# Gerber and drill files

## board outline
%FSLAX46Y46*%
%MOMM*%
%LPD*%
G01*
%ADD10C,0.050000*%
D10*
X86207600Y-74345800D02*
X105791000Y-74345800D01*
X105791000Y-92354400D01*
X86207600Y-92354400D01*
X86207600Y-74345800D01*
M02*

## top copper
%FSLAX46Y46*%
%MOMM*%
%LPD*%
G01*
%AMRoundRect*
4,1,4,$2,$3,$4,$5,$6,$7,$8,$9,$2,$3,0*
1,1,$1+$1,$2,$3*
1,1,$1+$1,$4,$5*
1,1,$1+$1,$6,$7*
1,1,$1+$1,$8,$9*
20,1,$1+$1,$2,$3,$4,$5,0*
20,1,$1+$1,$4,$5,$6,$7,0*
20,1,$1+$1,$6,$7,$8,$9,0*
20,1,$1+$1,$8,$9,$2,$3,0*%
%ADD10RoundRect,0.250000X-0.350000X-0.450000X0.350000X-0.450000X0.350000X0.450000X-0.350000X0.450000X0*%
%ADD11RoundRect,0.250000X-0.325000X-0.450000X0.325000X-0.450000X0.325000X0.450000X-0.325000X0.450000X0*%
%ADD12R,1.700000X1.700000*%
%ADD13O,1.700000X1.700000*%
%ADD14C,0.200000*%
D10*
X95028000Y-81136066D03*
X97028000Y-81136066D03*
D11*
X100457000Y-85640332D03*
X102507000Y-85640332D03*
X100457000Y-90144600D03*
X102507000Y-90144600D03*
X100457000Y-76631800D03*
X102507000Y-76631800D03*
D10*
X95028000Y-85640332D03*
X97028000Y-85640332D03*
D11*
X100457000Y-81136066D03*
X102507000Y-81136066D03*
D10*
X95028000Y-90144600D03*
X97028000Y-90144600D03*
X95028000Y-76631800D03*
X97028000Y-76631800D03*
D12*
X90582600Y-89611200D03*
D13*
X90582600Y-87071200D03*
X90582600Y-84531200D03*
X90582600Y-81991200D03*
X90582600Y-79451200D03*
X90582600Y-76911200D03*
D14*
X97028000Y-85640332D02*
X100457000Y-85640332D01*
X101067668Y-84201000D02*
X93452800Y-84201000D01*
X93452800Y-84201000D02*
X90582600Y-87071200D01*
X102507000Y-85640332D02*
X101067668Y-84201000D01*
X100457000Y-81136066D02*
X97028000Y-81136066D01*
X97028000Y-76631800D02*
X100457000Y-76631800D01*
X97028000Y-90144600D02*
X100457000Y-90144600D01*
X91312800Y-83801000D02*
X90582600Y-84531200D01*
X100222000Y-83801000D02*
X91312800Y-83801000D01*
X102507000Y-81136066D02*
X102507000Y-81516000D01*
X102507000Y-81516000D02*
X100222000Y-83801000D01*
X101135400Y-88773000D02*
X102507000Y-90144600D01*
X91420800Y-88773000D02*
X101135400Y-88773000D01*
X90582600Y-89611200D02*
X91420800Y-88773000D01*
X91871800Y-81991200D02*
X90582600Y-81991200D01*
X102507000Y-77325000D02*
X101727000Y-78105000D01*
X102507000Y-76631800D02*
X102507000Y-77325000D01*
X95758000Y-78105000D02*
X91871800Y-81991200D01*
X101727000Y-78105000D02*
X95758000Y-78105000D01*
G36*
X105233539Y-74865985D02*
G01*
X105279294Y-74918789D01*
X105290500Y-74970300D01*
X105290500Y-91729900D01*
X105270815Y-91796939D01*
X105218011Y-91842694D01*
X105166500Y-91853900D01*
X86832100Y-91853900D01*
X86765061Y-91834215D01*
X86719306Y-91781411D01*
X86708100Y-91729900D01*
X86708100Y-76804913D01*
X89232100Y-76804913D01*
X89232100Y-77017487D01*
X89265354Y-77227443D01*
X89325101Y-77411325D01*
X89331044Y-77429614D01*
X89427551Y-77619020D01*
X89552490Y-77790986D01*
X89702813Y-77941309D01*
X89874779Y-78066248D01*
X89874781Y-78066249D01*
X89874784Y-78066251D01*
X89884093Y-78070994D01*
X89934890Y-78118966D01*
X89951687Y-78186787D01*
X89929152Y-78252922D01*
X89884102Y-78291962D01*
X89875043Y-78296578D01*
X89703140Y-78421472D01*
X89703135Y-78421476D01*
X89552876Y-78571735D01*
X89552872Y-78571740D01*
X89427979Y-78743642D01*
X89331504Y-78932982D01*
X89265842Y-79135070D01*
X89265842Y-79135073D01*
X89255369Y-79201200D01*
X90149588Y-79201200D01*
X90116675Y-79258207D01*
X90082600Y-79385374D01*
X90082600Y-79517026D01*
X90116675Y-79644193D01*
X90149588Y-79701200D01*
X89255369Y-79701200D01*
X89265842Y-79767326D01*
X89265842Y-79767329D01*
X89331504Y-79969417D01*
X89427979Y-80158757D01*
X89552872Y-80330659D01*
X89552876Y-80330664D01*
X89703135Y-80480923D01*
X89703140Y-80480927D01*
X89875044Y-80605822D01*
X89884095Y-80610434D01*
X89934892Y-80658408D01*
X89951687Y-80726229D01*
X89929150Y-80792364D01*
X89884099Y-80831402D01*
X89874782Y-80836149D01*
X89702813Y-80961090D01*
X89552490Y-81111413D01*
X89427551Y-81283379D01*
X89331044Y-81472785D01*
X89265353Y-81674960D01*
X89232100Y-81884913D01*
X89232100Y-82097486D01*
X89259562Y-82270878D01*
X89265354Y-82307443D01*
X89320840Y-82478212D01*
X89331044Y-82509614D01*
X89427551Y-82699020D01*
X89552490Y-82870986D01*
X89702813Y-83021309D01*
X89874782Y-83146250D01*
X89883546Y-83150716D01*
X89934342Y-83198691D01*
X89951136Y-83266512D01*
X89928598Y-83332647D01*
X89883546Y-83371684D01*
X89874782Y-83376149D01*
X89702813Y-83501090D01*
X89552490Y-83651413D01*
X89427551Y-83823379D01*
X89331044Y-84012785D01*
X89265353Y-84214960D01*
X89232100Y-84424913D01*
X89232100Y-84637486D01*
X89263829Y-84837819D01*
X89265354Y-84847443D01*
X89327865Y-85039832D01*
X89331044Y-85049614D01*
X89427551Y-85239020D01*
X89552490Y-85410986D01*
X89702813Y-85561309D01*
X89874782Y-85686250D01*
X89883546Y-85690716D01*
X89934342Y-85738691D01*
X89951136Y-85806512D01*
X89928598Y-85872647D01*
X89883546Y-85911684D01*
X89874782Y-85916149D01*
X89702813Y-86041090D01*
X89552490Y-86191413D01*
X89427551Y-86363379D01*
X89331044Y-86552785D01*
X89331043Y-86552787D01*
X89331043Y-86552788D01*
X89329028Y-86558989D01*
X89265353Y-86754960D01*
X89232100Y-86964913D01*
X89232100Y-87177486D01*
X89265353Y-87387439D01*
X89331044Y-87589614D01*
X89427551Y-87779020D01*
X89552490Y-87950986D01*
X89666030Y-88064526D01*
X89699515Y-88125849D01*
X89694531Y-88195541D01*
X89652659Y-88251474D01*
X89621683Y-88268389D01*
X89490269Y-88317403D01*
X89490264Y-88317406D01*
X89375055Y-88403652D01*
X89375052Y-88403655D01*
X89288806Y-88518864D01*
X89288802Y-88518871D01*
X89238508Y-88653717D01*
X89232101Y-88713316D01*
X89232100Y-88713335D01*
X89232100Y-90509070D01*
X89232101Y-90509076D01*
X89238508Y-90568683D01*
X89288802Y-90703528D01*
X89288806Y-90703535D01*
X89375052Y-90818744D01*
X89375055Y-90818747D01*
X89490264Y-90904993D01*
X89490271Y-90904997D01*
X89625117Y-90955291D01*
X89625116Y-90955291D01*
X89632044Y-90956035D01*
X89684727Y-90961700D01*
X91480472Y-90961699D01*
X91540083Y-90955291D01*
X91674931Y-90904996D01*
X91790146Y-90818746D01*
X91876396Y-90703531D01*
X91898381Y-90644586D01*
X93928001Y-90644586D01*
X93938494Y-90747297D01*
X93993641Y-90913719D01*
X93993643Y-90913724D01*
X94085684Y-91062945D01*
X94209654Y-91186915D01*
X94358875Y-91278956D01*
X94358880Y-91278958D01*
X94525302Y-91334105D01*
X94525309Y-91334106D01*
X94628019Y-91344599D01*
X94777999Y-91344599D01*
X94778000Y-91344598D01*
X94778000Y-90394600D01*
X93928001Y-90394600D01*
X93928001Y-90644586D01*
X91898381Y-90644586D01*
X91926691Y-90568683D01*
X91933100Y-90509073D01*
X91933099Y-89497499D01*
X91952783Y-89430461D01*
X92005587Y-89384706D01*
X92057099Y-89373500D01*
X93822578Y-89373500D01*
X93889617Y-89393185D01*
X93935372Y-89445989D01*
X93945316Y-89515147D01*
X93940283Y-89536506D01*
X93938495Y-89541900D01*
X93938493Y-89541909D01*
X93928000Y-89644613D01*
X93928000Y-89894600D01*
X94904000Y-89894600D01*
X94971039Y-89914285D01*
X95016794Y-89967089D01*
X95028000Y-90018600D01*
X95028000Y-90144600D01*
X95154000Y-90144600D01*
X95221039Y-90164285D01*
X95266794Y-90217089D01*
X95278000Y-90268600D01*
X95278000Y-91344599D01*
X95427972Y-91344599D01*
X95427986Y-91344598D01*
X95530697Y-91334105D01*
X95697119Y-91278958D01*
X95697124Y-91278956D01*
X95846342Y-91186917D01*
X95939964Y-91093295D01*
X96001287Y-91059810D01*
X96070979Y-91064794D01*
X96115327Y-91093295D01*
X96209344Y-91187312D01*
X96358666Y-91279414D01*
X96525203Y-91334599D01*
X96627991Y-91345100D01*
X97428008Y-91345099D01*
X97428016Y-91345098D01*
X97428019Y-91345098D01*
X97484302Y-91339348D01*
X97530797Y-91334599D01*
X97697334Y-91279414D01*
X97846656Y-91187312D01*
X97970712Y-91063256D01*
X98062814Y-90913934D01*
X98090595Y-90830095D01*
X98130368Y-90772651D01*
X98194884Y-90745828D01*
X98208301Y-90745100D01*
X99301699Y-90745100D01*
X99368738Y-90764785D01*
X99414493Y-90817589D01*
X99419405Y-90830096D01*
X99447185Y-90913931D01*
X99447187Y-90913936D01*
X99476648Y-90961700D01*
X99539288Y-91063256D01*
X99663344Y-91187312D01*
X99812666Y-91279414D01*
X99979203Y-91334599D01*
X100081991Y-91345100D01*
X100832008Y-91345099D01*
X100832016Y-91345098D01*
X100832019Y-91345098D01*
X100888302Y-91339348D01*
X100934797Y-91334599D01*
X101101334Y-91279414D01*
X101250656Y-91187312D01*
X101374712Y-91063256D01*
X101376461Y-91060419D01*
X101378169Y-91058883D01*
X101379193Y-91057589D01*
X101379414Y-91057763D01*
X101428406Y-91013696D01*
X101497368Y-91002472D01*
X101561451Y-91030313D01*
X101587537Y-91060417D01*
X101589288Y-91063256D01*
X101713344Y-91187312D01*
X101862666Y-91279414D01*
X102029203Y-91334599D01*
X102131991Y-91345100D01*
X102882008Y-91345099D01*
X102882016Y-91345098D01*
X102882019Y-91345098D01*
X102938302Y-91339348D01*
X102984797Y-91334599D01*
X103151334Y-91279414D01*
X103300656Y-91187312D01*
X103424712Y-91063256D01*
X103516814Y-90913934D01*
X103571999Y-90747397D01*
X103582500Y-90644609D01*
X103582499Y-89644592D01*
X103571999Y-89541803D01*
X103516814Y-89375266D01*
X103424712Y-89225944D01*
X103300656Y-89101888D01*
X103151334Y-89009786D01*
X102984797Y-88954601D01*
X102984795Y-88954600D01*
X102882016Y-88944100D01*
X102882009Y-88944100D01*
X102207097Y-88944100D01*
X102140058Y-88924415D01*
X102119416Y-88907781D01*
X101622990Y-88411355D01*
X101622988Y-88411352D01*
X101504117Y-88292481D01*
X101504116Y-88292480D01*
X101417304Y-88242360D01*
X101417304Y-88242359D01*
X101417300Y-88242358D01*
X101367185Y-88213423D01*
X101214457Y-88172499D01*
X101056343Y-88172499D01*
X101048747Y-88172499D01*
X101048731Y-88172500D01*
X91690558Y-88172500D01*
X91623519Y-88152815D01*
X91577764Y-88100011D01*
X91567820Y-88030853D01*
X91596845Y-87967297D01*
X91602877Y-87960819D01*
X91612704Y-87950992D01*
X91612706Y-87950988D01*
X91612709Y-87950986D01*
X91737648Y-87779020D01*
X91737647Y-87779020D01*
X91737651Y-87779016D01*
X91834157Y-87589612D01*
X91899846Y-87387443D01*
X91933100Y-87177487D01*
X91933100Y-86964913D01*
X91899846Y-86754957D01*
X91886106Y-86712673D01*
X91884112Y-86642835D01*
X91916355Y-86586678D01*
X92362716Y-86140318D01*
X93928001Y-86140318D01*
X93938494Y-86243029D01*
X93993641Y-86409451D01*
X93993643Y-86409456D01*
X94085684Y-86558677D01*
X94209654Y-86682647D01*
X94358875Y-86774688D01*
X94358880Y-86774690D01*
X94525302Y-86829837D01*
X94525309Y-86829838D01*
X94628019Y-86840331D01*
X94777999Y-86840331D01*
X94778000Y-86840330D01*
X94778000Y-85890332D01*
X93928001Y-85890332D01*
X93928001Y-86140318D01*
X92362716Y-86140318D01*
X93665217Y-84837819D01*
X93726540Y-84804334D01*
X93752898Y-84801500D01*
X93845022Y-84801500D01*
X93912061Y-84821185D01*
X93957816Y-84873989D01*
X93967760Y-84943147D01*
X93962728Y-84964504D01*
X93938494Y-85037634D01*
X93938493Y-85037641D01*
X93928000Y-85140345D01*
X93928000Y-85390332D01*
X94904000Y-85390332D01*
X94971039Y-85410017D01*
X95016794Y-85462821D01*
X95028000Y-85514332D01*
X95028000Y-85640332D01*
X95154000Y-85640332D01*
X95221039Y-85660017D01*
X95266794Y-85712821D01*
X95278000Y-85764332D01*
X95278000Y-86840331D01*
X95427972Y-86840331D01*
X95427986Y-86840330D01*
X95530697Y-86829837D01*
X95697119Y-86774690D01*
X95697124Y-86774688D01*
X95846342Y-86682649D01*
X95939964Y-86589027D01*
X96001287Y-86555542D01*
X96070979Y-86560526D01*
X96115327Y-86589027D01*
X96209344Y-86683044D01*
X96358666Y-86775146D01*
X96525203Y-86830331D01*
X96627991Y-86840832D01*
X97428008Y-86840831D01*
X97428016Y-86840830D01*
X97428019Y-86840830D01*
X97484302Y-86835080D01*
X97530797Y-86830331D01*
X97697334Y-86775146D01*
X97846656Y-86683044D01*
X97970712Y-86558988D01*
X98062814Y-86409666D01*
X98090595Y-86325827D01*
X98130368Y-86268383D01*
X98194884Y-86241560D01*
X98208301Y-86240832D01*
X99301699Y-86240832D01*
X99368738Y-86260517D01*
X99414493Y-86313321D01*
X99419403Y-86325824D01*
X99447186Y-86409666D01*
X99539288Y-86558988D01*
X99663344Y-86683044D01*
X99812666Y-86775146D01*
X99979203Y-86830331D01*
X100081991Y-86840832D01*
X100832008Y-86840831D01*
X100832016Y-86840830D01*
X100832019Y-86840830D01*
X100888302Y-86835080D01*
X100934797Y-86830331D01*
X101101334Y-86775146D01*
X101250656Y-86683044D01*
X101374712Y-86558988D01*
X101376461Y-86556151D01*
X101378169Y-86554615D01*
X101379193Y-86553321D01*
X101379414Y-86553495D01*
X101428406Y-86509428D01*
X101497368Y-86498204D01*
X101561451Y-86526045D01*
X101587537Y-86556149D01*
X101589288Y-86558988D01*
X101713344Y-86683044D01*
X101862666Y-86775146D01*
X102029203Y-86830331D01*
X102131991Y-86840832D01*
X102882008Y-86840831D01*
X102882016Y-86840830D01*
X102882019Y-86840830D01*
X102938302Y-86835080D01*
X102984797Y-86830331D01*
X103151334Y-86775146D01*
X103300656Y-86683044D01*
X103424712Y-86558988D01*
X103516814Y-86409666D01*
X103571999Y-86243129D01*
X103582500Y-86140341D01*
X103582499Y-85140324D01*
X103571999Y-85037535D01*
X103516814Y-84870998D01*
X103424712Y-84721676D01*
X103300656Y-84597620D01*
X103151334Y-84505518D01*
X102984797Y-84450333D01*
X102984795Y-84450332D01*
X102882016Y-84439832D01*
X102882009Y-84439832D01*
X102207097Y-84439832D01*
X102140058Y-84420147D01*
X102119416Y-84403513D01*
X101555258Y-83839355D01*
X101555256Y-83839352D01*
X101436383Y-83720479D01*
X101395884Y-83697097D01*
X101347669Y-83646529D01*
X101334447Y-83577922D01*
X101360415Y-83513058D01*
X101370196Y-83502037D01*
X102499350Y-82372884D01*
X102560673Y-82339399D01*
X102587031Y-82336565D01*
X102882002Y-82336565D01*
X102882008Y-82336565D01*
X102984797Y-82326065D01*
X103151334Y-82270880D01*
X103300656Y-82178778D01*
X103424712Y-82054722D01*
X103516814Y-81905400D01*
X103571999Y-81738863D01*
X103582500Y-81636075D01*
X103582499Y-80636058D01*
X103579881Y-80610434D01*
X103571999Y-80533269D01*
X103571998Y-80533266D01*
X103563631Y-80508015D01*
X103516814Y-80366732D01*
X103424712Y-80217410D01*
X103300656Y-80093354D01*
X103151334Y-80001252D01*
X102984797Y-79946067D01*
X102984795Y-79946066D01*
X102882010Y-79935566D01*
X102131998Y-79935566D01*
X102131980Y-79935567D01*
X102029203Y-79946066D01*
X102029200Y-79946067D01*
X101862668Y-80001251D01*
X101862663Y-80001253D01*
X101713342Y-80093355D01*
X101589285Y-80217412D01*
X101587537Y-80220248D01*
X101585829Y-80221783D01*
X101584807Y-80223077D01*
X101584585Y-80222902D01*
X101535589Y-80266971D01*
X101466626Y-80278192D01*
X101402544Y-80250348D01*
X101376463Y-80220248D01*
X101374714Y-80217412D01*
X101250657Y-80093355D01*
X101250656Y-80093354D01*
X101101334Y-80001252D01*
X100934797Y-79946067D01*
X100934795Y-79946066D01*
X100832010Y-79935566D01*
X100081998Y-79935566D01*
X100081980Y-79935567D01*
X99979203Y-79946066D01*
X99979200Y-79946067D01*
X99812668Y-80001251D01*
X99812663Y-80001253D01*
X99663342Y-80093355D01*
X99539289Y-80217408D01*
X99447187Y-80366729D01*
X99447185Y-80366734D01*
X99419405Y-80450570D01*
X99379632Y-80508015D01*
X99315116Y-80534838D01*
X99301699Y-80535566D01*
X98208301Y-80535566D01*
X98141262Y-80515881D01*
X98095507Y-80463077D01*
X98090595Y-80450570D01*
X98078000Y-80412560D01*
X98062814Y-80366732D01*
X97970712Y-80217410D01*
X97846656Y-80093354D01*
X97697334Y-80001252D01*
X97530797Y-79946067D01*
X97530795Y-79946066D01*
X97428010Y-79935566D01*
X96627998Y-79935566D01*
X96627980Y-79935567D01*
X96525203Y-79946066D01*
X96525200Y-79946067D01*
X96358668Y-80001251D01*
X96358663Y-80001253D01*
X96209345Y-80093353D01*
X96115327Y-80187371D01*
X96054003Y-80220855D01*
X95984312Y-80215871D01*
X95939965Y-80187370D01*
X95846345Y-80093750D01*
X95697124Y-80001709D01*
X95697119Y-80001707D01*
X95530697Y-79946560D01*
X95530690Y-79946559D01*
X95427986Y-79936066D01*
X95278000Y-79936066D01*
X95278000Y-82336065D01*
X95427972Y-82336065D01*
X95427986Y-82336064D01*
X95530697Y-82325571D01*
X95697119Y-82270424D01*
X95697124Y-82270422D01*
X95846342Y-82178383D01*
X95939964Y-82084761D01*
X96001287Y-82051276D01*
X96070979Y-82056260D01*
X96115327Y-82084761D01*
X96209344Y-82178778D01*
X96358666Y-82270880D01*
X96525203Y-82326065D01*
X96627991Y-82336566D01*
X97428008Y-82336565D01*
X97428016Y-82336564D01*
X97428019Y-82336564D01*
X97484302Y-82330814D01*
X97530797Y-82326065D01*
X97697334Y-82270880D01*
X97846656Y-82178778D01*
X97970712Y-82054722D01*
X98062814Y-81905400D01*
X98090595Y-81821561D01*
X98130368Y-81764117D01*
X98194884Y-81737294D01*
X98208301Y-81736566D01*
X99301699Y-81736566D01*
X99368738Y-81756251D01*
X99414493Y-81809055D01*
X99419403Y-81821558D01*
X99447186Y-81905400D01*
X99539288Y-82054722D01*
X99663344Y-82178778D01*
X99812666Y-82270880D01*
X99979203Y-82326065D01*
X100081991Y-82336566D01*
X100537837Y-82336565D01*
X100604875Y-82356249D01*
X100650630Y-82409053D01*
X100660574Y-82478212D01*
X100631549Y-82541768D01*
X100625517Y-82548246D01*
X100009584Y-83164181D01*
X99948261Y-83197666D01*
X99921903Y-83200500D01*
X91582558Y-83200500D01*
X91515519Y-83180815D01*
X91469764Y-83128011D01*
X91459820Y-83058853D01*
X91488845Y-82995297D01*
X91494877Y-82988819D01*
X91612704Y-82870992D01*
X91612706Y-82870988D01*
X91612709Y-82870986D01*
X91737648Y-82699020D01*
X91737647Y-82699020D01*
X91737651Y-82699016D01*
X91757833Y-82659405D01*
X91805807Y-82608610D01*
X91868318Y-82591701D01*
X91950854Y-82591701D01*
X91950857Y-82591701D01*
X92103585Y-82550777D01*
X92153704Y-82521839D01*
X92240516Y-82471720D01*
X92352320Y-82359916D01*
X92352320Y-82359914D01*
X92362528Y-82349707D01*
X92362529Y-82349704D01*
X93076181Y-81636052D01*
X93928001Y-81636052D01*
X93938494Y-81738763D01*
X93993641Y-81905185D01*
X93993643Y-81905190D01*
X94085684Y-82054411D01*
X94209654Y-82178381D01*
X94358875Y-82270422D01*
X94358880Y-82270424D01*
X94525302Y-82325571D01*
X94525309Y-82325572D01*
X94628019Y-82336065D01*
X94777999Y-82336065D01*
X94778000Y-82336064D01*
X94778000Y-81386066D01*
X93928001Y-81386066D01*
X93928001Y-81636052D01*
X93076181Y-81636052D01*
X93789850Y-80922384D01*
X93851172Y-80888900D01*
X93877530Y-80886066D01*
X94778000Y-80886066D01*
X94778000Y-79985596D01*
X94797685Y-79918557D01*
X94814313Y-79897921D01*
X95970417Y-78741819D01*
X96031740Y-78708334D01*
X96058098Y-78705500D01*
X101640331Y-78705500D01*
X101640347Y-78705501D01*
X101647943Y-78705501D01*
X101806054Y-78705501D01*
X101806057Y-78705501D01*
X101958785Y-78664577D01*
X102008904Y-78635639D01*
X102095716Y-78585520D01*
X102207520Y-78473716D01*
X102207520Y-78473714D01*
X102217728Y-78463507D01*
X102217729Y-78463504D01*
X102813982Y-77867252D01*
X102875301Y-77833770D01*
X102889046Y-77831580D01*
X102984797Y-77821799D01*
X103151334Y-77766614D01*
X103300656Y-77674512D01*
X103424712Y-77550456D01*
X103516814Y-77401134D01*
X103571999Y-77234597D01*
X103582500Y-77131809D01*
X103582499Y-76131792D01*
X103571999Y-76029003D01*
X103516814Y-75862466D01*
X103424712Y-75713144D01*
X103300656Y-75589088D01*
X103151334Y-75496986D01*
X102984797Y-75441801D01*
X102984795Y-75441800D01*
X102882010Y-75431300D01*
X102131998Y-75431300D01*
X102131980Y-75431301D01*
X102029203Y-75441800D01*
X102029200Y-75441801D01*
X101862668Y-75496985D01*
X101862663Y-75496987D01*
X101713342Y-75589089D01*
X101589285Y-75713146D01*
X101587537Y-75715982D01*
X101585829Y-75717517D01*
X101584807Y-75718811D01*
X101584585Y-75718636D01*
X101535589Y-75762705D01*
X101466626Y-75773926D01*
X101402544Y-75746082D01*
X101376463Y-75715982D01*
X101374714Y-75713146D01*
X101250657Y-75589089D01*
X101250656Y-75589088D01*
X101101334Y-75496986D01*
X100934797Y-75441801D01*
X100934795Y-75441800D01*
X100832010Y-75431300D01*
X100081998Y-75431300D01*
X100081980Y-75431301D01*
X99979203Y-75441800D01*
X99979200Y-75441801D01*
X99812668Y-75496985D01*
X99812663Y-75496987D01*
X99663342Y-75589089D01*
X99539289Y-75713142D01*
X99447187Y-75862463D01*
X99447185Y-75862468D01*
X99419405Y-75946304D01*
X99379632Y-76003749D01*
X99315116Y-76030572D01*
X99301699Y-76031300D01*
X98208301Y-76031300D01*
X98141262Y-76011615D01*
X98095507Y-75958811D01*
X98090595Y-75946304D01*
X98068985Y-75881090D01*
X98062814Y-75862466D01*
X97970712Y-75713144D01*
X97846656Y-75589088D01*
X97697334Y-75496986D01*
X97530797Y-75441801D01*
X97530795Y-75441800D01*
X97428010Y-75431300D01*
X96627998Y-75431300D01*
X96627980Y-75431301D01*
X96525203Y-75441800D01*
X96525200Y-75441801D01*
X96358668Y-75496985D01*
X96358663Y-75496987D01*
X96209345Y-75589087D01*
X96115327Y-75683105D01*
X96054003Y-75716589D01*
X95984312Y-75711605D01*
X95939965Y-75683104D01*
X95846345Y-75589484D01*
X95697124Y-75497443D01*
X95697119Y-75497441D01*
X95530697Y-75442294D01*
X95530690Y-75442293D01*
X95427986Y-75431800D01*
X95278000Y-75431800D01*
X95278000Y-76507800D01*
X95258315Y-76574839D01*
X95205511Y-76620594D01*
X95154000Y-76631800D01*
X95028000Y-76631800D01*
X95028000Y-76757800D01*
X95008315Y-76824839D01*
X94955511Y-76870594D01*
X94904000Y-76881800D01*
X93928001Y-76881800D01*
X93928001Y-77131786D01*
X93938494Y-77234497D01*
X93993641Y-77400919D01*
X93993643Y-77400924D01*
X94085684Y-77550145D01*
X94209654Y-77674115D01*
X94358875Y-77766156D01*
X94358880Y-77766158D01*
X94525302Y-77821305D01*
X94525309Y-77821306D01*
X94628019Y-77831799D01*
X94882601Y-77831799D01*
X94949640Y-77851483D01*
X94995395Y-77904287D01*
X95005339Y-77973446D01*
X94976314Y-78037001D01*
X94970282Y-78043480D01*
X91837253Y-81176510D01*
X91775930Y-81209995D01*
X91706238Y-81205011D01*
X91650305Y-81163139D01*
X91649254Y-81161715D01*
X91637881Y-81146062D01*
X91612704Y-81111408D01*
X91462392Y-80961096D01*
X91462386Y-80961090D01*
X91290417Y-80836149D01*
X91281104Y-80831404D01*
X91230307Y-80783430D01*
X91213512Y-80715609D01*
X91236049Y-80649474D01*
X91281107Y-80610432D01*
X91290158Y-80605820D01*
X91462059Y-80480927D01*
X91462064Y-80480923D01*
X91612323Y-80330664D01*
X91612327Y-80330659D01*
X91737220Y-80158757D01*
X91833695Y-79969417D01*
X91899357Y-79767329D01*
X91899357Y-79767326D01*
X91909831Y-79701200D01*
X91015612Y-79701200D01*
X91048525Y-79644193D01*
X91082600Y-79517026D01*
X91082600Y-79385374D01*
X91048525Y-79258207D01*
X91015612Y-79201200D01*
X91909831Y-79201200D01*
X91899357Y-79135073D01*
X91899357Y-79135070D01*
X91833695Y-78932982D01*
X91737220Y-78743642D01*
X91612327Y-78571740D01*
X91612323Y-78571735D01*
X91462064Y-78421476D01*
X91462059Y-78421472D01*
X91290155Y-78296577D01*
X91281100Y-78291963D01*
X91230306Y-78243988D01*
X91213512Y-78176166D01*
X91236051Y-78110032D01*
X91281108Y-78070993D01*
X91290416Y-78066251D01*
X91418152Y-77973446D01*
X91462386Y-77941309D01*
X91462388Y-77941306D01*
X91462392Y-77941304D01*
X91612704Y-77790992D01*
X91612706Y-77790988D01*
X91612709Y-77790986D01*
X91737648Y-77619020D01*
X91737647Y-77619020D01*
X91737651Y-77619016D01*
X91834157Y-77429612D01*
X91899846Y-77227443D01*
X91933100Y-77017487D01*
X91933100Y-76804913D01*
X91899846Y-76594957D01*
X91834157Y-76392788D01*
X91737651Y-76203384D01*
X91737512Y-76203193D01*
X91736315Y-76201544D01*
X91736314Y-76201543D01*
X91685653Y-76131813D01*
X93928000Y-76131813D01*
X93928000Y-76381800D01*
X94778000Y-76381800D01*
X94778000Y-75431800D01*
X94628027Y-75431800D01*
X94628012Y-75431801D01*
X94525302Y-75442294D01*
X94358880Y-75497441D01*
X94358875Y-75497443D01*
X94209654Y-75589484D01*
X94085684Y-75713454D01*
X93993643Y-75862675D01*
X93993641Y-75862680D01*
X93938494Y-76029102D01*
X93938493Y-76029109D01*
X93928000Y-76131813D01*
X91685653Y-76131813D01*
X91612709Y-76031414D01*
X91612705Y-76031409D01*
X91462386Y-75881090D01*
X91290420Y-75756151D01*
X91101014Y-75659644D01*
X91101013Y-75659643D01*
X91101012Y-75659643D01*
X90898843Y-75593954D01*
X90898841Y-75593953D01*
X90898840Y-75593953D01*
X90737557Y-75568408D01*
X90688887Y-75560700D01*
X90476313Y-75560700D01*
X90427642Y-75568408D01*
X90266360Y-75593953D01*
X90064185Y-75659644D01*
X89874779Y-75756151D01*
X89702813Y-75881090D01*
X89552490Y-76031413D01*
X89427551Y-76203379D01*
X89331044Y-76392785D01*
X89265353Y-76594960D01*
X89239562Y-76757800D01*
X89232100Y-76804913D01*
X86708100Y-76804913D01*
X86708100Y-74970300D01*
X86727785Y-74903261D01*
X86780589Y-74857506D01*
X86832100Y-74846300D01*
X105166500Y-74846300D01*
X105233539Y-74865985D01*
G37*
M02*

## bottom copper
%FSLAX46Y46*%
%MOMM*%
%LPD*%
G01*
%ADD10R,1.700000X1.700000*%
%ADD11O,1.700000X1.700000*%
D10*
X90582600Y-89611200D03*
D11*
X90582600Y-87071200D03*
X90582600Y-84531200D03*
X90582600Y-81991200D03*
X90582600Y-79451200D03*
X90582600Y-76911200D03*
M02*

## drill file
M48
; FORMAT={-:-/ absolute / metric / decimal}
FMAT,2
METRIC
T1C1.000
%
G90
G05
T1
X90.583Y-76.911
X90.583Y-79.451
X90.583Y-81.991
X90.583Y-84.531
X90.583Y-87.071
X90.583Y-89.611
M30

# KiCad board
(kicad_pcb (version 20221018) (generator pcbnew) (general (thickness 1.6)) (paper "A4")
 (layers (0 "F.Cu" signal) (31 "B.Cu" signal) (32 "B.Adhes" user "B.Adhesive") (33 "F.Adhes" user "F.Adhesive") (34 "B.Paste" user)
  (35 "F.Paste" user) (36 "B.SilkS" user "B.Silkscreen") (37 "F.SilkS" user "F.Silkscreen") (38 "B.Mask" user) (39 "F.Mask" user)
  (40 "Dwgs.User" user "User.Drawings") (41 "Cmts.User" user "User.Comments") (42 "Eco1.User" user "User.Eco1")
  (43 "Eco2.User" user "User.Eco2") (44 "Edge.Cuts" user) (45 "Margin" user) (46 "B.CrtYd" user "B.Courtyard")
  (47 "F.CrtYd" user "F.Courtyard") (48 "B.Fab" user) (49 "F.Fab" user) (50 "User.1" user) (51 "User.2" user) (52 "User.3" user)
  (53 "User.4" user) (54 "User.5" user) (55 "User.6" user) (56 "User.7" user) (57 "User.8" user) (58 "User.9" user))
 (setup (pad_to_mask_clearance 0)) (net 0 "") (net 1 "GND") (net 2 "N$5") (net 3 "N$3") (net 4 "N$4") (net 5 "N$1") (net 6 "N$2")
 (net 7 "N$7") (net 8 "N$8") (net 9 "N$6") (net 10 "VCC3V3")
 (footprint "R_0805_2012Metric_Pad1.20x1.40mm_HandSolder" (layer "F.Cu") (at 96.028 81.136066)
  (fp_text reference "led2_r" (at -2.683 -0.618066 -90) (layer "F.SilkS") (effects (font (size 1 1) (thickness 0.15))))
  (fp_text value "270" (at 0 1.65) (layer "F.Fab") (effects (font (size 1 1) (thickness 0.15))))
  (pad "1" smd roundrect (at -1 0) (size 1.2 1.4) (layers "F.Cu" "F.Paste" "F.Mask") (roundrect_rratio 0.208333) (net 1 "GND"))
  (pad "2" smd roundrect (at 1 0) (size 1.2 1.4) (layers "F.Cu" "F.Paste" "F.Mask") (roundrect_rratio 0.208333) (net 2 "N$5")))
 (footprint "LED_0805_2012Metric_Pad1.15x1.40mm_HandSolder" (layer "F.Cu") (at 101.482 85.640332)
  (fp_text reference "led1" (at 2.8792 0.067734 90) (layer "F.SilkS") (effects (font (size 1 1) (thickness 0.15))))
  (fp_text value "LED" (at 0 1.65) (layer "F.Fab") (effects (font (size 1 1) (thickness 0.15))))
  (pad "1" smd roundrect (at -1.025 0) (size 1.15 1.4) (layers "F.Cu" "F.Paste" "F.Mask") (roundrect_rratio 0.217391) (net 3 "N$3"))
  (pad "2" smd roundrect (at 1.025 0) (size 1.15 1.4) (layers "F.Cu" "F.Paste" "F.Mask") (roundrect_rratio 0.217391) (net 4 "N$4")))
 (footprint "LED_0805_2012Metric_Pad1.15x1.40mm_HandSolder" (layer "F.Cu") (at 101.482 90.1446)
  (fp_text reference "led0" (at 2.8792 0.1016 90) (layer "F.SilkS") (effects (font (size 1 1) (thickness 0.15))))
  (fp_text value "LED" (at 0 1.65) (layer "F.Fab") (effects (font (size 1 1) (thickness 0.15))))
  (pad "1" smd roundrect (at -1.025 0) (size 1.15 1.4) (layers "F.Cu" "F.Paste" "F.Mask") (roundrect_rratio 0.217391) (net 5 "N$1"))
  (pad "2" smd roundrect (at 1.025 0) (size 1.15 1.4) (layers "F.Cu" "F.Paste" "F.Mask") (roundrect_rratio 0.217391) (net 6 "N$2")))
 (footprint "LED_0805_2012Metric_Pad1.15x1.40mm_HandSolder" (layer "F.Cu") (at 101.482 76.6318)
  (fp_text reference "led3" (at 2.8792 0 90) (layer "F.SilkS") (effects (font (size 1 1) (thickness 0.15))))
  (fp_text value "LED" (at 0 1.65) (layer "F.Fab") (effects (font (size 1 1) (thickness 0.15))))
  (pad "1" smd roundrect (at -1.025 0) (size 1.15 1.4) (layers "F.Cu" "F.Paste" "F.Mask") (roundrect_rratio 0.217391) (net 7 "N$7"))
  (pad "2" smd roundrect (at 1.025 0) (size 1.15 1.4) (layers "F.Cu" "F.Paste" "F.Mask") (roundrect_rratio 0.217391) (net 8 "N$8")))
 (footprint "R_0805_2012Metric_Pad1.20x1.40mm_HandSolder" (layer "F.Cu") (at 96.028 85.640332)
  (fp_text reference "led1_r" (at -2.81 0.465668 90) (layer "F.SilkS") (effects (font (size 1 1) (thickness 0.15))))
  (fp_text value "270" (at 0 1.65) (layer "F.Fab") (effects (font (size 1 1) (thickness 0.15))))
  (pad "1" smd roundrect (at -1 0) (size 1.2 1.4) (layers "F.Cu" "F.Paste" "F.Mask") (roundrect_rratio 0.208333) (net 1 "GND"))
  (pad "2" smd roundrect (at 1 0) (size 1.2 1.4) (layers "F.Cu" "F.Paste" "F.Mask") (roundrect_rratio 0.208333) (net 3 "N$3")))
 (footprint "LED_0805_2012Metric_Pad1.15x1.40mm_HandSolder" (layer "F.Cu") (at 101.482 81.136066)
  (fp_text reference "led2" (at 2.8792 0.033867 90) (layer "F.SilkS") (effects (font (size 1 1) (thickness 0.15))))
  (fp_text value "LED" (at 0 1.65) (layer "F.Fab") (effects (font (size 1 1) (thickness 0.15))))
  (pad "1" smd roundrect (at -1.025 0) (size 1.15 1.4) (layers "F.Cu" "F.Paste" "F.Mask") (roundrect_rratio 0.217391) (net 2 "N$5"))
  (pad "2" smd roundrect (at 1.025 0) (size 1.15 1.4) (layers "F.Cu" "F.Paste" "F.Mask") (roundrect_rratio 0.217391) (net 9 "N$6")))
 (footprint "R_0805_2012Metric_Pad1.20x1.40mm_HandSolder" (layer "F.Cu") (at 96.028 90.1446)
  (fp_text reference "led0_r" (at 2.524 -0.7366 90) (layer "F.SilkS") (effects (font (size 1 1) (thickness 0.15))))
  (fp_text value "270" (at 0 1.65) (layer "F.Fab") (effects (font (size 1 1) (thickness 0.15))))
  (pad "1" smd roundrect (at -1 0) (size 1.2 1.4) (layers "F.Cu" "F.Paste" "F.Mask") (roundrect_rratio 0.208333) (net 1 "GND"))
  (pad "2" smd roundrect (at 1 0) (size 1.2 1.4) (layers "F.Cu" "F.Paste" "F.Mask") (roundrect_rratio 0.208333) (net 5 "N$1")))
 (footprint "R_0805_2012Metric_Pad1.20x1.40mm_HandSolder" (layer "F.Cu") (at 96.028 76.6318)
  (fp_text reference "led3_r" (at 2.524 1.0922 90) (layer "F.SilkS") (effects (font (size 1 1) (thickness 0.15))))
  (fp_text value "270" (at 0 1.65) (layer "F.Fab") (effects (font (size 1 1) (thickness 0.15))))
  (pad "1" smd roundrect (at -1 0) (size 1.2 1.4) (layers "F.Cu" "F.Paste" "F.Mask") (roundrect_rratio 0.208333) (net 1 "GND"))
  (pad "2" smd roundrect (at 1 0) (size 1.2 1.4) (layers "F.Cu" "F.Paste" "F.Mask") (roundrect_rratio 0.208333) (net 7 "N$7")))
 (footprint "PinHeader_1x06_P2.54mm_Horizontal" (layer "F.Cu") (at 90.5826 89.6112 180)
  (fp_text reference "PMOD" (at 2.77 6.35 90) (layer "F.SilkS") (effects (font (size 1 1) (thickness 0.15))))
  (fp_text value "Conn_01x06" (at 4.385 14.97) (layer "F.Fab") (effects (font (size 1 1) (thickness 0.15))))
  (pad "1" thru_hole rect (at 0 0 180) (size 1.7 1.7) (drill 1) (layers "*.Cu" "*.Mask") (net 6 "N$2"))
  (pad "2" thru_hole oval (at 0 2.54 180) (size 1.7 1.7) (drill 1) (layers "*.Cu" "*.Mask") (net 4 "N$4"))
  (pad "3" thru_hole oval (at 0 5.08 180) (size 1.7 1.7) (drill 1) (layers "*.Cu" "*.Mask") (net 9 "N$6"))
  (pad "4" thru_hole oval (at 0 7.62 180) (size 1.7 1.7) (drill 1) (layers "*.Cu" "*.Mask") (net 8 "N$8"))
  (pad "5" thru_hole oval (at 0 10.16 180) (size 1.7 1.7) (drill 1) (layers "*.Cu" "*.Mask") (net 1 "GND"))
  (pad "6" thru_hole oval (at 0 12.7 180) (size 1.7 1.7) (drill 1) (layers "*.Cu" "*.Mask") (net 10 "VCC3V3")))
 (gr_rect (start 86.2076 74.3458) (end 105.791 92.3544) (stroke (width 0.05) (type default)) (fill none) (layer "Edge.Cuts"))
 (segment (start 97.028 85.640332) (end 100.457 85.640332) (width 0.2) (layer "F.Cu") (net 3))
 (segment (start 101.067668 84.201) (end 93.4528 84.201) (width 0.2) (layer "F.Cu") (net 4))
 (segment (start 93.4528 84.201) (end 90.5826 87.0712) (width 0.2) (layer "F.Cu") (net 4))
 (segment (start 102.507 85.640332) (end 101.067668 84.201) (width 0.2) (layer "F.Cu") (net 4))
 (segment (start 100.457 81.136066) (end 97.028 81.136066) (width 0.2) (layer "F.Cu") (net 2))
 (segment (start 97.028 76.6318) (end 100.457 76.6318) (width 0.2) (layer "F.Cu") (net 7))
 (segment (start 97.028 90.1446) (end 100.457 90.1446) (width 0.2) (layer "F.Cu") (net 5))
 (segment (start 91.3128 83.801) (end 90.5826 84.5312) (width 0.2) (layer "F.Cu") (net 9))
 (segment (start 100.222 83.801) (end 91.3128 83.801) (width 0.2) (layer "F.Cu") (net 9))
 (segment (start 102.507 81.136066) (end 102.507 81.516) (width 0.2) (layer "F.Cu") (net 9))
 (segment (start 102.507 81.516) (end 100.222 83.801) (width 0.2) (layer "F.Cu") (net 9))
 (segment (start 101.1354 88.773) (end 102.507 90.1446) (width 0.2) (layer "F.Cu") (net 6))
 (segment (start 91.4208 88.773) (end 101.1354 88.773) (width 0.2) (layer "F.Cu") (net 6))
 (segment (start 90.5826 89.6112) (end 91.4208 88.773) (width 0.2) (layer "F.Cu") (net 6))
 (segment (start 91.8718 81.9912) (end 90.5826 81.9912) (width 0.2) (layer "F.Cu") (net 8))
 (segment (start 102.507 77.325) (end 101.727 78.105) (width 0.2) (layer "F.Cu") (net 8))
 (segment (start 102.507 76.6318) (end 102.507 77.325) (width 0.2) (layer "F.Cu") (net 8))
 (segment (start 95.758 78.105) (end 91.8718 81.9912) (width 0.2) (layer "F.Cu") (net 8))
 (segment (start 101.727 78.105) (end 95.758 78.105) (width 0.2) (layer "F.Cu") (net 8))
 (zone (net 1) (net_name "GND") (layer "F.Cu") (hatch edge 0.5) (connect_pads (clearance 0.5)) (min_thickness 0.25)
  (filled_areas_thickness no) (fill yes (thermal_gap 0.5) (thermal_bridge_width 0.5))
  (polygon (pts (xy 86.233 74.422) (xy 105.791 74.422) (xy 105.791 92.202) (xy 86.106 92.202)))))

